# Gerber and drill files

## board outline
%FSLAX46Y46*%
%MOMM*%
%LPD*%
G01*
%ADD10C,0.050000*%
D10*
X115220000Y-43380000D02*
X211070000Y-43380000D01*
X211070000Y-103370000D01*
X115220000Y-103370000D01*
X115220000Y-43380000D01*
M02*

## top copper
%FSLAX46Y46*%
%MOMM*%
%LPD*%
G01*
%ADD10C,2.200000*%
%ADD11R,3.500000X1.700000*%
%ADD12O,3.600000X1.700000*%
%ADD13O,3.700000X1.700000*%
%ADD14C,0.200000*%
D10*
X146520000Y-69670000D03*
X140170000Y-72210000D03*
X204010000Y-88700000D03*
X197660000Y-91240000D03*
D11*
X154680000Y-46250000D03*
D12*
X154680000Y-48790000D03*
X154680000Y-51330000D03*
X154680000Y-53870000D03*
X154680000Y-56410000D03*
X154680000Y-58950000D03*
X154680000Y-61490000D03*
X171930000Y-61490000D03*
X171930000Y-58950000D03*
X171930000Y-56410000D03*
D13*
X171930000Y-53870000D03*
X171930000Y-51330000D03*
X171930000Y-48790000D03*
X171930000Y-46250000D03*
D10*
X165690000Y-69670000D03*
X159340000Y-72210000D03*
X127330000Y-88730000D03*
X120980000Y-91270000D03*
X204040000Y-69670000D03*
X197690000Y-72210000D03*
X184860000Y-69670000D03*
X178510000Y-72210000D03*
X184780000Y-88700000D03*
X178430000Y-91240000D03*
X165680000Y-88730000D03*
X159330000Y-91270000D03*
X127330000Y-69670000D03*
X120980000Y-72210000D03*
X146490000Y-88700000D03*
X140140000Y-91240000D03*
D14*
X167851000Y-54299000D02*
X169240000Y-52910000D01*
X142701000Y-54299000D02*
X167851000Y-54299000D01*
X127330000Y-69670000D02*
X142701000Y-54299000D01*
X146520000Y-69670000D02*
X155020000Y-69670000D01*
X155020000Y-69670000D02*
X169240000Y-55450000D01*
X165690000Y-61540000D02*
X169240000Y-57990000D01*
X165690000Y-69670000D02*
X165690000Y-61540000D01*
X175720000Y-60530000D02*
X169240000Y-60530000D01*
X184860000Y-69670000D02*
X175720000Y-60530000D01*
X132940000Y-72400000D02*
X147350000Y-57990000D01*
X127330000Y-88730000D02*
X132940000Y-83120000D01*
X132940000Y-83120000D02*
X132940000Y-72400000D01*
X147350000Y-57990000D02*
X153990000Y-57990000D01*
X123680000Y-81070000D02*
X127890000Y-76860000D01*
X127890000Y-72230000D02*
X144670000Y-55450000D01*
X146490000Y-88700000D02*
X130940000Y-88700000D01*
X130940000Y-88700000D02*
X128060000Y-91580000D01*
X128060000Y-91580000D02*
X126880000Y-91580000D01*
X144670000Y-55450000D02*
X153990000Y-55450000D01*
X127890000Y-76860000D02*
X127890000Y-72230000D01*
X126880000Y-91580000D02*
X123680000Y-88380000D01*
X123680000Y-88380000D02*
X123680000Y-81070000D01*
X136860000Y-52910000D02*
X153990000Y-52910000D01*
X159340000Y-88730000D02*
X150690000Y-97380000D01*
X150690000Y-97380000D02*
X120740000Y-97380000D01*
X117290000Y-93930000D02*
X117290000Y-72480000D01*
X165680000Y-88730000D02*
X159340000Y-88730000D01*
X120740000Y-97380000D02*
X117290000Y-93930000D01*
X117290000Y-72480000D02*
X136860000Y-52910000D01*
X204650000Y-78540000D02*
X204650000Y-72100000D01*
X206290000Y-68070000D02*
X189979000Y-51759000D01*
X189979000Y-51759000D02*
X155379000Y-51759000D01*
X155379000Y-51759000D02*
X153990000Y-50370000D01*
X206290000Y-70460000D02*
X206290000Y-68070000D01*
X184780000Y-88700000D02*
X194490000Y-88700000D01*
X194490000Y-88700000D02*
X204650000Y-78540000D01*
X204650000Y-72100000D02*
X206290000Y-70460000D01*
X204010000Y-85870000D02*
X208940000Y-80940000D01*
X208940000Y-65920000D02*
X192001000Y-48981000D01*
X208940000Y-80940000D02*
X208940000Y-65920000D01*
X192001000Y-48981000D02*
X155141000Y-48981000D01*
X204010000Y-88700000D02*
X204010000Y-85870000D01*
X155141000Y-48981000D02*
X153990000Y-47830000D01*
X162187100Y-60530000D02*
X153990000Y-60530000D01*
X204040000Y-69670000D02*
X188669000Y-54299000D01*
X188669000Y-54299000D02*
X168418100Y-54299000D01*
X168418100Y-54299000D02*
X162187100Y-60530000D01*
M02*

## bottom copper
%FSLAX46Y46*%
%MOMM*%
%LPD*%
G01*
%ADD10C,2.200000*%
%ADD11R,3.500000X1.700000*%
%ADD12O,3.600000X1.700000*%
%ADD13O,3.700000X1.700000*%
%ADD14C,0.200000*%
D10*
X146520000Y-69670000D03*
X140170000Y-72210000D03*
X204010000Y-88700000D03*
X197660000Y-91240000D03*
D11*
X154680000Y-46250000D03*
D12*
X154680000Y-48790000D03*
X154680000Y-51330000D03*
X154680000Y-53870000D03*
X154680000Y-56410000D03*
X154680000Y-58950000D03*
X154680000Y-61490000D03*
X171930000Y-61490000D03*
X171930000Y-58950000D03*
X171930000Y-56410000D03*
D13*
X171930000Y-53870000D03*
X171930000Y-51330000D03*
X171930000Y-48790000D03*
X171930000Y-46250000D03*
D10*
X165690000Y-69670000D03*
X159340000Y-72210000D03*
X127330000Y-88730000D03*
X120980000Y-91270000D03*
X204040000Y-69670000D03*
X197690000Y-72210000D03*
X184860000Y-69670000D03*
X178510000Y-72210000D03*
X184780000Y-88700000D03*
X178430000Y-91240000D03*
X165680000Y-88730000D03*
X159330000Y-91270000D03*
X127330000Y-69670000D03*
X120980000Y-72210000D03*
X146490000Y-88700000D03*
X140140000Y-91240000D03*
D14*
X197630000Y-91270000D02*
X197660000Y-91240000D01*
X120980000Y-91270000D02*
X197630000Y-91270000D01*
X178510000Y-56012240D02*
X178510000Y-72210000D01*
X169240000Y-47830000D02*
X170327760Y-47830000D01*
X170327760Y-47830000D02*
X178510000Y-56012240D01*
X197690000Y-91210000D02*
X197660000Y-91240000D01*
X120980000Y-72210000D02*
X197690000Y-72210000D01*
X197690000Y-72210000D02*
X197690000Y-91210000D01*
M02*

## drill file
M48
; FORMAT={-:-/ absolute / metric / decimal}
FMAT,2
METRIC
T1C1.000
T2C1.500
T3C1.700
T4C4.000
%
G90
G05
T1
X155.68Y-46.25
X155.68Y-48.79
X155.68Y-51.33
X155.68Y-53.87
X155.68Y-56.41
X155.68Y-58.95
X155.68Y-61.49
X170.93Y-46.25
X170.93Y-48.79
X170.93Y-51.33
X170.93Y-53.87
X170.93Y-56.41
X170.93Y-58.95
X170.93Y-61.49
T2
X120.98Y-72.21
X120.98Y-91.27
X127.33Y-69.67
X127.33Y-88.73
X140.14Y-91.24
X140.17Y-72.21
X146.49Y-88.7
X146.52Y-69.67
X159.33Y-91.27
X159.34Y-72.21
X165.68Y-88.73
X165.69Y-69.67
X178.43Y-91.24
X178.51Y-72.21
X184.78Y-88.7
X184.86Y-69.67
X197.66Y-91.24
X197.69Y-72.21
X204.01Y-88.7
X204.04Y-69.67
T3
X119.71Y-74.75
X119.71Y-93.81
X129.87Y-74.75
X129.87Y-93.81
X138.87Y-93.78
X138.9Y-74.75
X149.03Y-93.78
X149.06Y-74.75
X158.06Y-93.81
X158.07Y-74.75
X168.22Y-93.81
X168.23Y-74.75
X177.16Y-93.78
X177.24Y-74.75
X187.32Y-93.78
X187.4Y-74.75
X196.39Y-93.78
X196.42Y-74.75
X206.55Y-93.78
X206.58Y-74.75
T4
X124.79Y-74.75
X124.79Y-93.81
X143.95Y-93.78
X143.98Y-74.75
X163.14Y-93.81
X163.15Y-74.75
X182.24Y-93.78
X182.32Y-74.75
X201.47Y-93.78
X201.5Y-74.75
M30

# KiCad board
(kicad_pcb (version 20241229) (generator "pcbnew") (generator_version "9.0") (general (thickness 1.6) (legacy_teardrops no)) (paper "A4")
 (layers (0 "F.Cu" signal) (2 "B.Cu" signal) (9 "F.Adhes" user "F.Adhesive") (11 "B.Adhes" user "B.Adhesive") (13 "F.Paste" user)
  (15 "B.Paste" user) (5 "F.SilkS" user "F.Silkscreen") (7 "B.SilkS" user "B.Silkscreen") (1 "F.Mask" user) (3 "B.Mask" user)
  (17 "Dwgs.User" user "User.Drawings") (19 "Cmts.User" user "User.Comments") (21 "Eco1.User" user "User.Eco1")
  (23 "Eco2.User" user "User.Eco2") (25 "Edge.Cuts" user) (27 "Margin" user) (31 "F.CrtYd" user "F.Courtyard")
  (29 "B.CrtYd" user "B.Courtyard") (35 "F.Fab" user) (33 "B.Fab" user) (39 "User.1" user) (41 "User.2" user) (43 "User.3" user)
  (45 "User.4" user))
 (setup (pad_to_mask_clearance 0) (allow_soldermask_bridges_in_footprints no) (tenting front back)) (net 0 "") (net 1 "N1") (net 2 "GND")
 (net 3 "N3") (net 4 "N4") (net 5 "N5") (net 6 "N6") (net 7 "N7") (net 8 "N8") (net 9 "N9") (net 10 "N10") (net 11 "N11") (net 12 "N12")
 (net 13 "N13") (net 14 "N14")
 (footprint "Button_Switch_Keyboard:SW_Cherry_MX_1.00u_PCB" (layer "F.Cu") (at 146.52 69.67)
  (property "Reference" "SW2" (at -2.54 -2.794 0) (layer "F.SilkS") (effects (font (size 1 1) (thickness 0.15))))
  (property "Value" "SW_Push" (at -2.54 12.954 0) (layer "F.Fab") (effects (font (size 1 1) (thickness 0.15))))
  (pad "" np_thru_hole circle (at -7.62 5.08) (size 1.7 1.7) (drill 1.7) (layers "*.Cu" "*.Mask"))
  (pad "" np_thru_hole circle (at -2.54 5.08) (size 4 4) (drill 4) (layers "*.Cu" "*.Mask"))
  (pad "" np_thru_hole circle (at 2.54 5.08) (size 1.7 1.7) (drill 1.7) (layers "*.Cu" "*.Mask"))
  (pad "1" thru_hole circle (at 0 0) (size 2.2 2.2) (drill 1.5) (layers "*.Cu" "*.Mask") (remove_unused_layers no) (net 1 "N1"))
  (pad "2" thru_hole circle (at -6.35 2.54) (size 2.2 2.2) (drill 1.5) (layers "*.Cu" "*.Mask") (remove_unused_layers no) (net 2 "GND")))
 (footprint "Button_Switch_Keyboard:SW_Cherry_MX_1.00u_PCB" (layer "F.Cu") (at 204.01 88.7)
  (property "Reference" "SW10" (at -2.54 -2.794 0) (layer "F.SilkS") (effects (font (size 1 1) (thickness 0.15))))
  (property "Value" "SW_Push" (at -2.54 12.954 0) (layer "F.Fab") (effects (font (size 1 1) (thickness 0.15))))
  (pad "" np_thru_hole circle (at -7.62 5.08) (size 1.7 1.7) (drill 1.7) (layers "*.Cu" "*.Mask"))
  (pad "" np_thru_hole circle (at -2.54 5.08) (size 4 4) (drill 4) (layers "*.Cu" "*.Mask"))
  (pad "" np_thru_hole circle (at 2.54 5.08) (size 1.7 1.7) (drill 1.7) (layers "*.Cu" "*.Mask"))
  (pad "1" thru_hole circle (at 0 0) (size 2.2 2.2) (drill 1.5) (layers "*.Cu" "*.Mask") (remove_unused_layers no) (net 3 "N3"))
  (pad "2" thru_hole circle (at -6.35 2.54) (size 2.2 2.2) (drill 1.5) (layers "*.Cu" "*.Mask") (remove_unused_layers no) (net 2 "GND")))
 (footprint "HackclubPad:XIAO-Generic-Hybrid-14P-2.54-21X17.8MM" (layer "F.Cu") (at 163.305 53.87)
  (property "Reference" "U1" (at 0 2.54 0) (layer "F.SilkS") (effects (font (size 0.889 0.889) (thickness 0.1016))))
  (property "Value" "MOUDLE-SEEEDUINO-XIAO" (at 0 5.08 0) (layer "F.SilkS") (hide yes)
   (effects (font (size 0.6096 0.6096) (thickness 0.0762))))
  (pad "1" thru_hole rect (at -7.625 -7.62) (size 3.5 1.7) (drill 1 (offset -1 0)) (layers "*.Cu" "*.Mask") (remove_unused_layers no)
   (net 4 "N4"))
  (pad "2" thru_hole oval (at -7.625 -5.08) (size 3.6 1.7) (drill 1 (offset -1 0)) (layers "*.Cu" "*.Mask") (remove_unused_layers no)
   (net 3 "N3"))
  (pad "3" thru_hole oval (at -7.625 -2.54) (size 3.6 1.7) (drill 1 (offset -1 0)) (layers "*.Cu" "*.Mask") (remove_unused_layers no)
   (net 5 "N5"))
  (pad "4" thru_hole oval (at -7.625 0) (size 3.6 1.7) (drill 1 (offset -1 0)) (layers "*.Cu" "*.Mask") (remove_unused_layers no)
   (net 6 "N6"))
  (pad "5" thru_hole oval (at -7.625 2.54) (size 3.6 1.7) (drill 1 (offset -1 0)) (layers "*.Cu" "*.Mask") (remove_unused_layers no)
   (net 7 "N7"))
  (pad "6" thru_hole oval (at -7.625 5.08 180) (size 3.6 1.7) (drill 1 (offset 1 0)) (layers "*.Cu" "*.Mask") (remove_unused_layers no)
   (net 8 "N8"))
  (pad "7" thru_hole oval (at -7.625 7.62) (size 3.6 1.7) (drill 1 (offset -1 0)) (layers "*.Cu" "*.Mask") (remove_unused_layers no)
   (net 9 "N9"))
  (pad "8" thru_hole oval (at 7.625 7.62) (size 3.6 1.7) (drill 1 (offset 1 0)) (layers "*.Cu" "*.Mask") (remove_unused_layers no)
   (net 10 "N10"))
  (pad "9" thru_hole oval (at 7.625 5.08) (size 3.6 1.7) (drill 1 (offset 1 0)) (layers "*.Cu" "*.Mask") (remove_unused_layers no)
   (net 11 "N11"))
  (pad "10" thru_hole oval (at 7.625 2.54) (size 3.6 1.7) (drill 1 (offset 1 0)) (layers "*.Cu" "*.Mask") (remove_unused_layers no)
   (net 1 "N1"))
  (pad "11" thru_hole oval (at 7.625 0) (size 3.7 1.7) (drill 1 (offset 1 0)) (layers "*.Cu" "*.Mask") (remove_unused_layers no)
   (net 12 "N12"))
  (pad "12" thru_hole oval (at 7.625 -2.54) (size 3.7 1.7) (drill 1 (offset 1 0)) (layers "*.Cu" "*.Mask") (remove_unused_layers no)
   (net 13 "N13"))
  (pad "13" thru_hole oval (at 7.625 -5.08) (size 3.7 1.7) (drill 1 (offset 1 0)) (layers "*.Cu" "*.Mask") (remove_unused_layers no)
   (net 2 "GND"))
  (pad "14" thru_hole oval (at 7.625 -7.62) (size 3.7 1.7) (drill 1 (offset 1 0)) (layers "*.Cu" "*.Mask") (remove_unused_layers no)
   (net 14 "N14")))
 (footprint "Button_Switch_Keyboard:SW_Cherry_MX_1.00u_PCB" (layer "F.Cu") (at 165.69 69.67)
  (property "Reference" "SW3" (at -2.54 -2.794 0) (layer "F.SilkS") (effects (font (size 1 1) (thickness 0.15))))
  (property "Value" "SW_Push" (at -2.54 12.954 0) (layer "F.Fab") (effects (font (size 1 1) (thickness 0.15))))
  (pad "" np_thru_hole circle (at -7.62 5.08) (size 1.7 1.7) (drill 1.7) (layers "*.Cu" "*.Mask"))
  (pad "" np_thru_hole circle (at -2.54 5.08) (size 4 4) (drill 4) (layers "*.Cu" "*.Mask"))
  (pad "" np_thru_hole circle (at 2.54 5.08) (size 1.7 1.7) (drill 1.7) (layers "*.Cu" "*.Mask"))
  (pad "1" thru_hole circle (at 0 0) (size 2.2 2.2) (drill 1.5) (layers "*.Cu" "*.Mask") (remove_unused_layers no) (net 11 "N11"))
  (pad "2" thru_hole circle (at -6.35 2.54) (size 2.2 2.2) (drill 1.5) (layers "*.Cu" "*.Mask") (remove_unused_layers no) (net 2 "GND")))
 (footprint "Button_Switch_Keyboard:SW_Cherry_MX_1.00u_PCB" (layer "F.Cu") (at 127.33 88.73)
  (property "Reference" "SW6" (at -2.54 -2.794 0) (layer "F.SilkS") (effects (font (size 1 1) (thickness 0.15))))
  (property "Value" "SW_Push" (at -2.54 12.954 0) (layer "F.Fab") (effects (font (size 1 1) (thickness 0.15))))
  (pad "" np_thru_hole circle (at -7.62 5.08) (size 1.7 1.7) (drill 1.7) (layers "*.Cu" "*.Mask"))
  (pad "" np_thru_hole circle (at -2.54 5.08) (size 4 4) (drill 4) (layers "*.Cu" "*.Mask"))
  (pad "" np_thru_hole circle (at 2.54 5.08) (size 1.7 1.7) (drill 1.7) (layers "*.Cu" "*.Mask"))
  (pad "1" thru_hole circle (at 0 0) (size 2.2 2.2) (drill 1.5) (layers "*.Cu" "*.Mask") (remove_unused_layers no) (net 8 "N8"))
  (pad "2" thru_hole circle (at -6.35 2.54) (size 2.2 2.2) (drill 1.5) (layers "*.Cu" "*.Mask") (remove_unused_layers no) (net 2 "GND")))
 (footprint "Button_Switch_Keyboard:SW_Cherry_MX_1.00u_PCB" (layer "F.Cu") (at 204.04 69.67)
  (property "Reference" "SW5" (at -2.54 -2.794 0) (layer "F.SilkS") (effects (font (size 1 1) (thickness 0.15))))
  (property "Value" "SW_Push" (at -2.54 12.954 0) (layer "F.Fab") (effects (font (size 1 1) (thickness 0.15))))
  (pad "" np_thru_hole circle (at -7.62 5.08) (size 1.7 1.7) (drill 1.7) (layers "*.Cu" "*.Mask"))
  (pad "" np_thru_hole circle (at -2.54 5.08) (size 4 4) (drill 4) (layers "*.Cu" "*.Mask"))
  (pad "" np_thru_hole circle (at 2.54 5.08) (size 1.7 1.7) (drill 1.7) (layers "*.Cu" "*.Mask"))
  (pad "1" thru_hole circle (at 0 0) (size 2.2 2.2) (drill 1.5) (layers "*.Cu" "*.Mask") (remove_unused_layers no) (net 9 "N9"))
  (pad "2" thru_hole circle (at -6.35 2.54) (size 2.2 2.2) (drill 1.5) (layers "*.Cu" "*.Mask") (remove_unused_layers no) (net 2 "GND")))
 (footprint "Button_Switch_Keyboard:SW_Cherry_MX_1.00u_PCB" (layer "F.Cu") (at 184.86 69.67)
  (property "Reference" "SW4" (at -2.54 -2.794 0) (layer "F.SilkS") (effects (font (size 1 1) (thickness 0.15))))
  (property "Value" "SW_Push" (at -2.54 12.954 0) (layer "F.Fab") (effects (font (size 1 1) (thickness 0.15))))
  (pad "" np_thru_hole circle (at -7.62 5.08) (size 1.7 1.7) (drill 1.7) (layers "*.Cu" "*.Mask"))
  (pad "" np_thru_hole circle (at -2.54 5.08) (size 4 4) (drill 4) (layers "*.Cu" "*.Mask"))
  (pad "" np_thru_hole circle (at 2.54 5.08) (size 1.7 1.7) (drill 1.7) (layers "*.Cu" "*.Mask"))
  (pad "1" thru_hole circle (at 0 0) (size 2.2 2.2) (drill 1.5) (layers "*.Cu" "*.Mask") (remove_unused_layers no) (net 10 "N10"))
  (pad "2" thru_hole circle (at -6.35 2.54) (size 2.2 2.2) (drill 1.5) (layers "*.Cu" "*.Mask") (remove_unused_layers no) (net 2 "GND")))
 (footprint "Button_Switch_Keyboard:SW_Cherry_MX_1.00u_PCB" (layer "F.Cu") (at 184.78 88.7)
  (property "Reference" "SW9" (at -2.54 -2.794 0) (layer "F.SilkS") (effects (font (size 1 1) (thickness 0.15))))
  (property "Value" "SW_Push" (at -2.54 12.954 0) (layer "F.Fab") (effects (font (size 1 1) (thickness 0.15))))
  (pad "" np_thru_hole circle (at -7.62 5.08) (size 1.7 1.7) (drill 1.7) (layers "*.Cu" "*.Mask"))
  (pad "" np_thru_hole circle (at -2.54 5.08) (size 4 4) (drill 4) (layers "*.Cu" "*.Mask"))
  (pad "" np_thru_hole circle (at 2.54 5.08) (size 1.7 1.7) (drill 1.7) (layers "*.Cu" "*.Mask"))
  (pad "1" thru_hole circle (at 0 0) (size 2.2 2.2) (drill 1.5) (layers "*.Cu" "*.Mask") (remove_unused_layers no) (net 5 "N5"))
  (pad "2" thru_hole circle (at -6.35 2.54) (size 2.2 2.2) (drill 1.5) (layers "*.Cu" "*.Mask") (remove_unused_layers no) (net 2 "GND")))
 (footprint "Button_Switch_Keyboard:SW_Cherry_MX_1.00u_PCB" (layer "F.Cu") (at 165.68 88.73)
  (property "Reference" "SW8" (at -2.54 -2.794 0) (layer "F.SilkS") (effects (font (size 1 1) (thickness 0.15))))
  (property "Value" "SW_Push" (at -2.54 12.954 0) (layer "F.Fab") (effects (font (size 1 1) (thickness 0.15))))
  (pad "" np_thru_hole circle (at -7.62 5.08) (size 1.7 1.7) (drill 1.7) (layers "*.Cu" "*.Mask"))
  (pad "" np_thru_hole circle (at -2.54 5.08) (size 4 4) (drill 4) (layers "*.Cu" "*.Mask"))
  (pad "" np_thru_hole circle (at 2.54 5.08) (size 1.7 1.7) (drill 1.7) (layers "*.Cu" "*.Mask"))
  (pad "1" thru_hole circle (at 0 0) (size 2.2 2.2) (drill 1.5) (layers "*.Cu" "*.Mask") (remove_unused_layers no) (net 6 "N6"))
  (pad "2" thru_hole circle (at -6.35 2.54) (size 2.2 2.2) (drill 1.5) (layers "*.Cu" "*.Mask") (remove_unused_layers no) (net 2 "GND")))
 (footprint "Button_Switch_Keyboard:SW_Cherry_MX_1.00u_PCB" (layer "F.Cu") (at 127.33 69.67)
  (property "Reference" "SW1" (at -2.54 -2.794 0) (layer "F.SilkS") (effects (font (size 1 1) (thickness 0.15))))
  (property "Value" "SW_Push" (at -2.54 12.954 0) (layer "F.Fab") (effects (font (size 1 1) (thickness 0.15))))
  (pad "" np_thru_hole circle (at -7.62 5.08) (size 1.7 1.7) (drill 1.7) (layers "*.Cu" "*.Mask"))
  (pad "" np_thru_hole circle (at -2.54 5.08) (size 4 4) (drill 4) (layers "*.Cu" "*.Mask"))
  (pad "" np_thru_hole circle (at 2.54 5.08) (size 1.7 1.7) (drill 1.7) (layers "*.Cu" "*.Mask"))
  (pad "1" thru_hole circle (at 0 0) (size 2.2 2.2) (drill 1.5) (layers "*.Cu" "*.Mask") (remove_unused_layers no) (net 12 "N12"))
  (pad "2" thru_hole circle (at -6.35 2.54) (size 2.2 2.2) (drill 1.5) (layers "*.Cu" "*.Mask") (remove_unused_layers no) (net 2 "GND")))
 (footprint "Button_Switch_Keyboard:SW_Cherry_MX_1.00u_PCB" (layer "F.Cu") (at 146.49 88.7)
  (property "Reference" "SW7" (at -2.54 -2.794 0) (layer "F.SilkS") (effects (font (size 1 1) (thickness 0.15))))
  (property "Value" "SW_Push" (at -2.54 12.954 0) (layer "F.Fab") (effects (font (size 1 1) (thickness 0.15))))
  (pad "" np_thru_hole circle (at -7.62 5.08) (size 1.7 1.7) (drill 1.7) (layers "*.Cu" "*.Mask"))
  (pad "" np_thru_hole circle (at -2.54 5.08) (size 4 4) (drill 4) (layers "*.Cu" "*.Mask"))
  (pad "" np_thru_hole circle (at 2.54 5.08) (size 1.7 1.7) (drill 1.7) (layers "*.Cu" "*.Mask"))
  (pad "1" thru_hole circle (at 0 0) (size 2.2 2.2) (drill 1.5) (layers "*.Cu" "*.Mask") (remove_unused_layers no) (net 7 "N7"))
  (pad "2" thru_hole circle (at -6.35 2.54) (size 2.2 2.2) (drill 1.5) (layers "*.Cu" "*.Mask") (remove_unused_layers no) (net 2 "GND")))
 (gr_rect (start 115.22 43.38) (end 211.07 103.37) (stroke (width 0.05) (type default)) (fill no) (layer "Edge.Cuts"))
 (segment (start 197.63 91.27) (end 197.66 91.24) (width 0.2) (layer "B.Cu") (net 2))
 (segment (start 120.98 91.27) (end 197.63 91.27) (width 0.2) (layer "B.Cu") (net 2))
 (segment (start 178.51 56.01224) (end 178.51 72.21) (width 0.2) (layer "B.Cu") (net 2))
 (segment (start 169.24 47.83) (end 170.32776 47.83) (width 0.2) (layer "B.Cu") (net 2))
 (segment (start 170.32776 47.83) (end 178.51 56.01224) (width 0.2) (layer "B.Cu") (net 2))
 (segment (start 197.69 91.21) (end 197.66 91.24) (width 0.2) (layer "B.Cu") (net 2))
 (segment (start 120.98 72.21) (end 197.69 72.21) (width 0.2) (layer "B.Cu") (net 2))
 (segment (start 197.69 72.21) (end 197.69 91.21) (width 0.2) (layer "B.Cu") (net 2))
 (segment (start 167.851 54.299) (end 169.24 52.91) (width 0.2) (layer "F.Cu") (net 12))
 (segment (start 142.701 54.299) (end 167.851 54.299) (width 0.2) (layer "F.Cu") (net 12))
 (segment (start 127.33 69.67) (end 142.701 54.299) (width 0.2) (layer "F.Cu") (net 12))
 (segment (start 146.52 69.67) (end 155.02 69.67) (width 0.2) (layer "F.Cu") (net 1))
 (segment (start 155.02 69.67) (end 169.24 55.45) (width 0.2) (layer "F.Cu") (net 1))
 (segment (start 165.69 61.54) (end 169.24 57.99) (width 0.2) (layer "F.Cu") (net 11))
 (segment (start 165.69 69.67) (end 165.69 61.54) (width 0.2) (layer "F.Cu") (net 11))
 (segment (start 175.72 60.53) (end 169.24 60.53) (width 0.2) (layer "F.Cu") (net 10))
 (segment (start 184.86 69.67) (end 175.72 60.53) (width 0.2) (layer "F.Cu") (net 10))
 (segment (start 132.94 72.4) (end 147.35 57.99) (width 0.2) (layer "F.Cu") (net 8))
 (segment (start 127.33 88.73) (end 132.94 83.12) (width 0.2) (layer "F.Cu") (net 8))
 (segment (start 132.94 83.12) (end 132.94 72.4) (width 0.2) (layer "F.Cu") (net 8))
 (segment (start 147.35 57.99) (end 153.99 57.99) (width 0.2) (layer "F.Cu") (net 8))
 (segment (start 123.68 81.07) (end 127.89 76.86) (width 0.2) (layer "F.Cu") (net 7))
 (segment (start 127.89 72.23) (end 144.67 55.45) (width 0.2) (layer "F.Cu") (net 7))
 (segment (start 146.49 88.7) (end 130.94 88.7) (width 0.2) (layer "F.Cu") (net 7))
 (segment (start 130.94 88.7) (end 128.06 91.58) (width 0.2) (layer "F.Cu") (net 7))
 (segment (start 128.06 91.58) (end 126.88 91.58) (width 0.2) (layer "F.Cu") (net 7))
 (segment (start 144.67 55.45) (end 153.99 55.45) (width 0.2) (layer "F.Cu") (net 7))
 (segment (start 127.89 76.86) (end 127.89 72.23) (width 0.2) (layer "F.Cu") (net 7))
 (segment (start 126.88 91.58) (end 123.68 88.38) (width 0.2) (layer "F.Cu") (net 7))
 (segment (start 123.68 88.38) (end 123.68 81.07) (width 0.2) (layer "F.Cu") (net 7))
 (segment (start 136.86 52.91) (end 153.99 52.91) (width 0.2) (layer "F.Cu") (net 6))
 (segment (start 159.34 88.73) (end 150.69 97.38) (width 0.2) (layer "F.Cu") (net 6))
 (segment (start 150.69 97.38) (end 120.74 97.38) (width 0.2) (layer "F.Cu") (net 6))
 (segment (start 117.29 93.93) (end 117.29 72.48) (width 0.2) (layer "F.Cu") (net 6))
 (segment (start 165.68 88.73) (end 159.34 88.73) (width 0.2) (layer "F.Cu") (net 6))
 (segment (start 120.74 97.38) (end 117.29 93.93) (width 0.2) (layer "F.Cu") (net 6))
 (segment (start 117.29 72.48) (end 136.86 52.91) (width 0.2) (layer "F.Cu") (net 6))
 (segment (start 204.65 78.54) (end 204.65 72.1) (width 0.2) (layer "F.Cu") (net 5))
 (segment (start 206.29 68.07) (end 189.979 51.759) (width 0.2) (layer "F.Cu") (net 5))
 (segment (start 189.979 51.759) (end 155.379 51.759) (width 0.2) (layer "F.Cu") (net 5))
 (segment (start 155.379 51.759) (end 153.99 50.37) (width 0.2) (layer "F.Cu") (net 5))
 (segment (start 206.29 70.46) (end 206.29 68.07) (width 0.2) (layer "F.Cu") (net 5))
 (segment (start 184.78 88.7) (end 194.49 88.7) (width 0.2) (layer "F.Cu") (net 5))
 (segment (start 194.49 88.7) (end 204.65 78.54) (width 0.2) (layer "F.Cu") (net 5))
 (segment (start 204.65 72.1) (end 206.29 70.46) (width 0.2) (layer "F.Cu") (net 5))
 (segment (start 204.01 85.87) (end 208.94 80.94) (width 0.2) (layer "F.Cu") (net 3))
 (segment (start 208.94 65.92) (end 192.001 48.981) (width 0.2) (layer "F.Cu") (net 3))
 (segment (start 208.94 80.94) (end 208.94 65.92) (width 0.2) (layer "F.Cu") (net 3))
 (segment (start 192.001 48.981) (end 155.141 48.981) (width 0.2) (layer "F.Cu") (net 3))
 (segment (start 204.01 88.7) (end 204.01 85.87) (width 0.2) (layer "F.Cu") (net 3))
 (segment (start 155.141 48.981) (end 153.99 47.83) (width 0.2) (layer "F.Cu") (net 3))
 (segment (start 162.1871 60.53) (end 153.99 60.53) (width 0.2) (layer "F.Cu") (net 9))
 (segment (start 204.04 69.67) (end 188.669 54.299) (width 0.2) (layer "F.Cu") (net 9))
 (segment (start 188.669 54.299) (end 168.4181 54.299) (width 0.2) (layer "F.Cu") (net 9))
 (segment (start 168.4181 54.299) (end 162.1871 60.53) (width 0.2) (layer "F.Cu") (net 9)))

